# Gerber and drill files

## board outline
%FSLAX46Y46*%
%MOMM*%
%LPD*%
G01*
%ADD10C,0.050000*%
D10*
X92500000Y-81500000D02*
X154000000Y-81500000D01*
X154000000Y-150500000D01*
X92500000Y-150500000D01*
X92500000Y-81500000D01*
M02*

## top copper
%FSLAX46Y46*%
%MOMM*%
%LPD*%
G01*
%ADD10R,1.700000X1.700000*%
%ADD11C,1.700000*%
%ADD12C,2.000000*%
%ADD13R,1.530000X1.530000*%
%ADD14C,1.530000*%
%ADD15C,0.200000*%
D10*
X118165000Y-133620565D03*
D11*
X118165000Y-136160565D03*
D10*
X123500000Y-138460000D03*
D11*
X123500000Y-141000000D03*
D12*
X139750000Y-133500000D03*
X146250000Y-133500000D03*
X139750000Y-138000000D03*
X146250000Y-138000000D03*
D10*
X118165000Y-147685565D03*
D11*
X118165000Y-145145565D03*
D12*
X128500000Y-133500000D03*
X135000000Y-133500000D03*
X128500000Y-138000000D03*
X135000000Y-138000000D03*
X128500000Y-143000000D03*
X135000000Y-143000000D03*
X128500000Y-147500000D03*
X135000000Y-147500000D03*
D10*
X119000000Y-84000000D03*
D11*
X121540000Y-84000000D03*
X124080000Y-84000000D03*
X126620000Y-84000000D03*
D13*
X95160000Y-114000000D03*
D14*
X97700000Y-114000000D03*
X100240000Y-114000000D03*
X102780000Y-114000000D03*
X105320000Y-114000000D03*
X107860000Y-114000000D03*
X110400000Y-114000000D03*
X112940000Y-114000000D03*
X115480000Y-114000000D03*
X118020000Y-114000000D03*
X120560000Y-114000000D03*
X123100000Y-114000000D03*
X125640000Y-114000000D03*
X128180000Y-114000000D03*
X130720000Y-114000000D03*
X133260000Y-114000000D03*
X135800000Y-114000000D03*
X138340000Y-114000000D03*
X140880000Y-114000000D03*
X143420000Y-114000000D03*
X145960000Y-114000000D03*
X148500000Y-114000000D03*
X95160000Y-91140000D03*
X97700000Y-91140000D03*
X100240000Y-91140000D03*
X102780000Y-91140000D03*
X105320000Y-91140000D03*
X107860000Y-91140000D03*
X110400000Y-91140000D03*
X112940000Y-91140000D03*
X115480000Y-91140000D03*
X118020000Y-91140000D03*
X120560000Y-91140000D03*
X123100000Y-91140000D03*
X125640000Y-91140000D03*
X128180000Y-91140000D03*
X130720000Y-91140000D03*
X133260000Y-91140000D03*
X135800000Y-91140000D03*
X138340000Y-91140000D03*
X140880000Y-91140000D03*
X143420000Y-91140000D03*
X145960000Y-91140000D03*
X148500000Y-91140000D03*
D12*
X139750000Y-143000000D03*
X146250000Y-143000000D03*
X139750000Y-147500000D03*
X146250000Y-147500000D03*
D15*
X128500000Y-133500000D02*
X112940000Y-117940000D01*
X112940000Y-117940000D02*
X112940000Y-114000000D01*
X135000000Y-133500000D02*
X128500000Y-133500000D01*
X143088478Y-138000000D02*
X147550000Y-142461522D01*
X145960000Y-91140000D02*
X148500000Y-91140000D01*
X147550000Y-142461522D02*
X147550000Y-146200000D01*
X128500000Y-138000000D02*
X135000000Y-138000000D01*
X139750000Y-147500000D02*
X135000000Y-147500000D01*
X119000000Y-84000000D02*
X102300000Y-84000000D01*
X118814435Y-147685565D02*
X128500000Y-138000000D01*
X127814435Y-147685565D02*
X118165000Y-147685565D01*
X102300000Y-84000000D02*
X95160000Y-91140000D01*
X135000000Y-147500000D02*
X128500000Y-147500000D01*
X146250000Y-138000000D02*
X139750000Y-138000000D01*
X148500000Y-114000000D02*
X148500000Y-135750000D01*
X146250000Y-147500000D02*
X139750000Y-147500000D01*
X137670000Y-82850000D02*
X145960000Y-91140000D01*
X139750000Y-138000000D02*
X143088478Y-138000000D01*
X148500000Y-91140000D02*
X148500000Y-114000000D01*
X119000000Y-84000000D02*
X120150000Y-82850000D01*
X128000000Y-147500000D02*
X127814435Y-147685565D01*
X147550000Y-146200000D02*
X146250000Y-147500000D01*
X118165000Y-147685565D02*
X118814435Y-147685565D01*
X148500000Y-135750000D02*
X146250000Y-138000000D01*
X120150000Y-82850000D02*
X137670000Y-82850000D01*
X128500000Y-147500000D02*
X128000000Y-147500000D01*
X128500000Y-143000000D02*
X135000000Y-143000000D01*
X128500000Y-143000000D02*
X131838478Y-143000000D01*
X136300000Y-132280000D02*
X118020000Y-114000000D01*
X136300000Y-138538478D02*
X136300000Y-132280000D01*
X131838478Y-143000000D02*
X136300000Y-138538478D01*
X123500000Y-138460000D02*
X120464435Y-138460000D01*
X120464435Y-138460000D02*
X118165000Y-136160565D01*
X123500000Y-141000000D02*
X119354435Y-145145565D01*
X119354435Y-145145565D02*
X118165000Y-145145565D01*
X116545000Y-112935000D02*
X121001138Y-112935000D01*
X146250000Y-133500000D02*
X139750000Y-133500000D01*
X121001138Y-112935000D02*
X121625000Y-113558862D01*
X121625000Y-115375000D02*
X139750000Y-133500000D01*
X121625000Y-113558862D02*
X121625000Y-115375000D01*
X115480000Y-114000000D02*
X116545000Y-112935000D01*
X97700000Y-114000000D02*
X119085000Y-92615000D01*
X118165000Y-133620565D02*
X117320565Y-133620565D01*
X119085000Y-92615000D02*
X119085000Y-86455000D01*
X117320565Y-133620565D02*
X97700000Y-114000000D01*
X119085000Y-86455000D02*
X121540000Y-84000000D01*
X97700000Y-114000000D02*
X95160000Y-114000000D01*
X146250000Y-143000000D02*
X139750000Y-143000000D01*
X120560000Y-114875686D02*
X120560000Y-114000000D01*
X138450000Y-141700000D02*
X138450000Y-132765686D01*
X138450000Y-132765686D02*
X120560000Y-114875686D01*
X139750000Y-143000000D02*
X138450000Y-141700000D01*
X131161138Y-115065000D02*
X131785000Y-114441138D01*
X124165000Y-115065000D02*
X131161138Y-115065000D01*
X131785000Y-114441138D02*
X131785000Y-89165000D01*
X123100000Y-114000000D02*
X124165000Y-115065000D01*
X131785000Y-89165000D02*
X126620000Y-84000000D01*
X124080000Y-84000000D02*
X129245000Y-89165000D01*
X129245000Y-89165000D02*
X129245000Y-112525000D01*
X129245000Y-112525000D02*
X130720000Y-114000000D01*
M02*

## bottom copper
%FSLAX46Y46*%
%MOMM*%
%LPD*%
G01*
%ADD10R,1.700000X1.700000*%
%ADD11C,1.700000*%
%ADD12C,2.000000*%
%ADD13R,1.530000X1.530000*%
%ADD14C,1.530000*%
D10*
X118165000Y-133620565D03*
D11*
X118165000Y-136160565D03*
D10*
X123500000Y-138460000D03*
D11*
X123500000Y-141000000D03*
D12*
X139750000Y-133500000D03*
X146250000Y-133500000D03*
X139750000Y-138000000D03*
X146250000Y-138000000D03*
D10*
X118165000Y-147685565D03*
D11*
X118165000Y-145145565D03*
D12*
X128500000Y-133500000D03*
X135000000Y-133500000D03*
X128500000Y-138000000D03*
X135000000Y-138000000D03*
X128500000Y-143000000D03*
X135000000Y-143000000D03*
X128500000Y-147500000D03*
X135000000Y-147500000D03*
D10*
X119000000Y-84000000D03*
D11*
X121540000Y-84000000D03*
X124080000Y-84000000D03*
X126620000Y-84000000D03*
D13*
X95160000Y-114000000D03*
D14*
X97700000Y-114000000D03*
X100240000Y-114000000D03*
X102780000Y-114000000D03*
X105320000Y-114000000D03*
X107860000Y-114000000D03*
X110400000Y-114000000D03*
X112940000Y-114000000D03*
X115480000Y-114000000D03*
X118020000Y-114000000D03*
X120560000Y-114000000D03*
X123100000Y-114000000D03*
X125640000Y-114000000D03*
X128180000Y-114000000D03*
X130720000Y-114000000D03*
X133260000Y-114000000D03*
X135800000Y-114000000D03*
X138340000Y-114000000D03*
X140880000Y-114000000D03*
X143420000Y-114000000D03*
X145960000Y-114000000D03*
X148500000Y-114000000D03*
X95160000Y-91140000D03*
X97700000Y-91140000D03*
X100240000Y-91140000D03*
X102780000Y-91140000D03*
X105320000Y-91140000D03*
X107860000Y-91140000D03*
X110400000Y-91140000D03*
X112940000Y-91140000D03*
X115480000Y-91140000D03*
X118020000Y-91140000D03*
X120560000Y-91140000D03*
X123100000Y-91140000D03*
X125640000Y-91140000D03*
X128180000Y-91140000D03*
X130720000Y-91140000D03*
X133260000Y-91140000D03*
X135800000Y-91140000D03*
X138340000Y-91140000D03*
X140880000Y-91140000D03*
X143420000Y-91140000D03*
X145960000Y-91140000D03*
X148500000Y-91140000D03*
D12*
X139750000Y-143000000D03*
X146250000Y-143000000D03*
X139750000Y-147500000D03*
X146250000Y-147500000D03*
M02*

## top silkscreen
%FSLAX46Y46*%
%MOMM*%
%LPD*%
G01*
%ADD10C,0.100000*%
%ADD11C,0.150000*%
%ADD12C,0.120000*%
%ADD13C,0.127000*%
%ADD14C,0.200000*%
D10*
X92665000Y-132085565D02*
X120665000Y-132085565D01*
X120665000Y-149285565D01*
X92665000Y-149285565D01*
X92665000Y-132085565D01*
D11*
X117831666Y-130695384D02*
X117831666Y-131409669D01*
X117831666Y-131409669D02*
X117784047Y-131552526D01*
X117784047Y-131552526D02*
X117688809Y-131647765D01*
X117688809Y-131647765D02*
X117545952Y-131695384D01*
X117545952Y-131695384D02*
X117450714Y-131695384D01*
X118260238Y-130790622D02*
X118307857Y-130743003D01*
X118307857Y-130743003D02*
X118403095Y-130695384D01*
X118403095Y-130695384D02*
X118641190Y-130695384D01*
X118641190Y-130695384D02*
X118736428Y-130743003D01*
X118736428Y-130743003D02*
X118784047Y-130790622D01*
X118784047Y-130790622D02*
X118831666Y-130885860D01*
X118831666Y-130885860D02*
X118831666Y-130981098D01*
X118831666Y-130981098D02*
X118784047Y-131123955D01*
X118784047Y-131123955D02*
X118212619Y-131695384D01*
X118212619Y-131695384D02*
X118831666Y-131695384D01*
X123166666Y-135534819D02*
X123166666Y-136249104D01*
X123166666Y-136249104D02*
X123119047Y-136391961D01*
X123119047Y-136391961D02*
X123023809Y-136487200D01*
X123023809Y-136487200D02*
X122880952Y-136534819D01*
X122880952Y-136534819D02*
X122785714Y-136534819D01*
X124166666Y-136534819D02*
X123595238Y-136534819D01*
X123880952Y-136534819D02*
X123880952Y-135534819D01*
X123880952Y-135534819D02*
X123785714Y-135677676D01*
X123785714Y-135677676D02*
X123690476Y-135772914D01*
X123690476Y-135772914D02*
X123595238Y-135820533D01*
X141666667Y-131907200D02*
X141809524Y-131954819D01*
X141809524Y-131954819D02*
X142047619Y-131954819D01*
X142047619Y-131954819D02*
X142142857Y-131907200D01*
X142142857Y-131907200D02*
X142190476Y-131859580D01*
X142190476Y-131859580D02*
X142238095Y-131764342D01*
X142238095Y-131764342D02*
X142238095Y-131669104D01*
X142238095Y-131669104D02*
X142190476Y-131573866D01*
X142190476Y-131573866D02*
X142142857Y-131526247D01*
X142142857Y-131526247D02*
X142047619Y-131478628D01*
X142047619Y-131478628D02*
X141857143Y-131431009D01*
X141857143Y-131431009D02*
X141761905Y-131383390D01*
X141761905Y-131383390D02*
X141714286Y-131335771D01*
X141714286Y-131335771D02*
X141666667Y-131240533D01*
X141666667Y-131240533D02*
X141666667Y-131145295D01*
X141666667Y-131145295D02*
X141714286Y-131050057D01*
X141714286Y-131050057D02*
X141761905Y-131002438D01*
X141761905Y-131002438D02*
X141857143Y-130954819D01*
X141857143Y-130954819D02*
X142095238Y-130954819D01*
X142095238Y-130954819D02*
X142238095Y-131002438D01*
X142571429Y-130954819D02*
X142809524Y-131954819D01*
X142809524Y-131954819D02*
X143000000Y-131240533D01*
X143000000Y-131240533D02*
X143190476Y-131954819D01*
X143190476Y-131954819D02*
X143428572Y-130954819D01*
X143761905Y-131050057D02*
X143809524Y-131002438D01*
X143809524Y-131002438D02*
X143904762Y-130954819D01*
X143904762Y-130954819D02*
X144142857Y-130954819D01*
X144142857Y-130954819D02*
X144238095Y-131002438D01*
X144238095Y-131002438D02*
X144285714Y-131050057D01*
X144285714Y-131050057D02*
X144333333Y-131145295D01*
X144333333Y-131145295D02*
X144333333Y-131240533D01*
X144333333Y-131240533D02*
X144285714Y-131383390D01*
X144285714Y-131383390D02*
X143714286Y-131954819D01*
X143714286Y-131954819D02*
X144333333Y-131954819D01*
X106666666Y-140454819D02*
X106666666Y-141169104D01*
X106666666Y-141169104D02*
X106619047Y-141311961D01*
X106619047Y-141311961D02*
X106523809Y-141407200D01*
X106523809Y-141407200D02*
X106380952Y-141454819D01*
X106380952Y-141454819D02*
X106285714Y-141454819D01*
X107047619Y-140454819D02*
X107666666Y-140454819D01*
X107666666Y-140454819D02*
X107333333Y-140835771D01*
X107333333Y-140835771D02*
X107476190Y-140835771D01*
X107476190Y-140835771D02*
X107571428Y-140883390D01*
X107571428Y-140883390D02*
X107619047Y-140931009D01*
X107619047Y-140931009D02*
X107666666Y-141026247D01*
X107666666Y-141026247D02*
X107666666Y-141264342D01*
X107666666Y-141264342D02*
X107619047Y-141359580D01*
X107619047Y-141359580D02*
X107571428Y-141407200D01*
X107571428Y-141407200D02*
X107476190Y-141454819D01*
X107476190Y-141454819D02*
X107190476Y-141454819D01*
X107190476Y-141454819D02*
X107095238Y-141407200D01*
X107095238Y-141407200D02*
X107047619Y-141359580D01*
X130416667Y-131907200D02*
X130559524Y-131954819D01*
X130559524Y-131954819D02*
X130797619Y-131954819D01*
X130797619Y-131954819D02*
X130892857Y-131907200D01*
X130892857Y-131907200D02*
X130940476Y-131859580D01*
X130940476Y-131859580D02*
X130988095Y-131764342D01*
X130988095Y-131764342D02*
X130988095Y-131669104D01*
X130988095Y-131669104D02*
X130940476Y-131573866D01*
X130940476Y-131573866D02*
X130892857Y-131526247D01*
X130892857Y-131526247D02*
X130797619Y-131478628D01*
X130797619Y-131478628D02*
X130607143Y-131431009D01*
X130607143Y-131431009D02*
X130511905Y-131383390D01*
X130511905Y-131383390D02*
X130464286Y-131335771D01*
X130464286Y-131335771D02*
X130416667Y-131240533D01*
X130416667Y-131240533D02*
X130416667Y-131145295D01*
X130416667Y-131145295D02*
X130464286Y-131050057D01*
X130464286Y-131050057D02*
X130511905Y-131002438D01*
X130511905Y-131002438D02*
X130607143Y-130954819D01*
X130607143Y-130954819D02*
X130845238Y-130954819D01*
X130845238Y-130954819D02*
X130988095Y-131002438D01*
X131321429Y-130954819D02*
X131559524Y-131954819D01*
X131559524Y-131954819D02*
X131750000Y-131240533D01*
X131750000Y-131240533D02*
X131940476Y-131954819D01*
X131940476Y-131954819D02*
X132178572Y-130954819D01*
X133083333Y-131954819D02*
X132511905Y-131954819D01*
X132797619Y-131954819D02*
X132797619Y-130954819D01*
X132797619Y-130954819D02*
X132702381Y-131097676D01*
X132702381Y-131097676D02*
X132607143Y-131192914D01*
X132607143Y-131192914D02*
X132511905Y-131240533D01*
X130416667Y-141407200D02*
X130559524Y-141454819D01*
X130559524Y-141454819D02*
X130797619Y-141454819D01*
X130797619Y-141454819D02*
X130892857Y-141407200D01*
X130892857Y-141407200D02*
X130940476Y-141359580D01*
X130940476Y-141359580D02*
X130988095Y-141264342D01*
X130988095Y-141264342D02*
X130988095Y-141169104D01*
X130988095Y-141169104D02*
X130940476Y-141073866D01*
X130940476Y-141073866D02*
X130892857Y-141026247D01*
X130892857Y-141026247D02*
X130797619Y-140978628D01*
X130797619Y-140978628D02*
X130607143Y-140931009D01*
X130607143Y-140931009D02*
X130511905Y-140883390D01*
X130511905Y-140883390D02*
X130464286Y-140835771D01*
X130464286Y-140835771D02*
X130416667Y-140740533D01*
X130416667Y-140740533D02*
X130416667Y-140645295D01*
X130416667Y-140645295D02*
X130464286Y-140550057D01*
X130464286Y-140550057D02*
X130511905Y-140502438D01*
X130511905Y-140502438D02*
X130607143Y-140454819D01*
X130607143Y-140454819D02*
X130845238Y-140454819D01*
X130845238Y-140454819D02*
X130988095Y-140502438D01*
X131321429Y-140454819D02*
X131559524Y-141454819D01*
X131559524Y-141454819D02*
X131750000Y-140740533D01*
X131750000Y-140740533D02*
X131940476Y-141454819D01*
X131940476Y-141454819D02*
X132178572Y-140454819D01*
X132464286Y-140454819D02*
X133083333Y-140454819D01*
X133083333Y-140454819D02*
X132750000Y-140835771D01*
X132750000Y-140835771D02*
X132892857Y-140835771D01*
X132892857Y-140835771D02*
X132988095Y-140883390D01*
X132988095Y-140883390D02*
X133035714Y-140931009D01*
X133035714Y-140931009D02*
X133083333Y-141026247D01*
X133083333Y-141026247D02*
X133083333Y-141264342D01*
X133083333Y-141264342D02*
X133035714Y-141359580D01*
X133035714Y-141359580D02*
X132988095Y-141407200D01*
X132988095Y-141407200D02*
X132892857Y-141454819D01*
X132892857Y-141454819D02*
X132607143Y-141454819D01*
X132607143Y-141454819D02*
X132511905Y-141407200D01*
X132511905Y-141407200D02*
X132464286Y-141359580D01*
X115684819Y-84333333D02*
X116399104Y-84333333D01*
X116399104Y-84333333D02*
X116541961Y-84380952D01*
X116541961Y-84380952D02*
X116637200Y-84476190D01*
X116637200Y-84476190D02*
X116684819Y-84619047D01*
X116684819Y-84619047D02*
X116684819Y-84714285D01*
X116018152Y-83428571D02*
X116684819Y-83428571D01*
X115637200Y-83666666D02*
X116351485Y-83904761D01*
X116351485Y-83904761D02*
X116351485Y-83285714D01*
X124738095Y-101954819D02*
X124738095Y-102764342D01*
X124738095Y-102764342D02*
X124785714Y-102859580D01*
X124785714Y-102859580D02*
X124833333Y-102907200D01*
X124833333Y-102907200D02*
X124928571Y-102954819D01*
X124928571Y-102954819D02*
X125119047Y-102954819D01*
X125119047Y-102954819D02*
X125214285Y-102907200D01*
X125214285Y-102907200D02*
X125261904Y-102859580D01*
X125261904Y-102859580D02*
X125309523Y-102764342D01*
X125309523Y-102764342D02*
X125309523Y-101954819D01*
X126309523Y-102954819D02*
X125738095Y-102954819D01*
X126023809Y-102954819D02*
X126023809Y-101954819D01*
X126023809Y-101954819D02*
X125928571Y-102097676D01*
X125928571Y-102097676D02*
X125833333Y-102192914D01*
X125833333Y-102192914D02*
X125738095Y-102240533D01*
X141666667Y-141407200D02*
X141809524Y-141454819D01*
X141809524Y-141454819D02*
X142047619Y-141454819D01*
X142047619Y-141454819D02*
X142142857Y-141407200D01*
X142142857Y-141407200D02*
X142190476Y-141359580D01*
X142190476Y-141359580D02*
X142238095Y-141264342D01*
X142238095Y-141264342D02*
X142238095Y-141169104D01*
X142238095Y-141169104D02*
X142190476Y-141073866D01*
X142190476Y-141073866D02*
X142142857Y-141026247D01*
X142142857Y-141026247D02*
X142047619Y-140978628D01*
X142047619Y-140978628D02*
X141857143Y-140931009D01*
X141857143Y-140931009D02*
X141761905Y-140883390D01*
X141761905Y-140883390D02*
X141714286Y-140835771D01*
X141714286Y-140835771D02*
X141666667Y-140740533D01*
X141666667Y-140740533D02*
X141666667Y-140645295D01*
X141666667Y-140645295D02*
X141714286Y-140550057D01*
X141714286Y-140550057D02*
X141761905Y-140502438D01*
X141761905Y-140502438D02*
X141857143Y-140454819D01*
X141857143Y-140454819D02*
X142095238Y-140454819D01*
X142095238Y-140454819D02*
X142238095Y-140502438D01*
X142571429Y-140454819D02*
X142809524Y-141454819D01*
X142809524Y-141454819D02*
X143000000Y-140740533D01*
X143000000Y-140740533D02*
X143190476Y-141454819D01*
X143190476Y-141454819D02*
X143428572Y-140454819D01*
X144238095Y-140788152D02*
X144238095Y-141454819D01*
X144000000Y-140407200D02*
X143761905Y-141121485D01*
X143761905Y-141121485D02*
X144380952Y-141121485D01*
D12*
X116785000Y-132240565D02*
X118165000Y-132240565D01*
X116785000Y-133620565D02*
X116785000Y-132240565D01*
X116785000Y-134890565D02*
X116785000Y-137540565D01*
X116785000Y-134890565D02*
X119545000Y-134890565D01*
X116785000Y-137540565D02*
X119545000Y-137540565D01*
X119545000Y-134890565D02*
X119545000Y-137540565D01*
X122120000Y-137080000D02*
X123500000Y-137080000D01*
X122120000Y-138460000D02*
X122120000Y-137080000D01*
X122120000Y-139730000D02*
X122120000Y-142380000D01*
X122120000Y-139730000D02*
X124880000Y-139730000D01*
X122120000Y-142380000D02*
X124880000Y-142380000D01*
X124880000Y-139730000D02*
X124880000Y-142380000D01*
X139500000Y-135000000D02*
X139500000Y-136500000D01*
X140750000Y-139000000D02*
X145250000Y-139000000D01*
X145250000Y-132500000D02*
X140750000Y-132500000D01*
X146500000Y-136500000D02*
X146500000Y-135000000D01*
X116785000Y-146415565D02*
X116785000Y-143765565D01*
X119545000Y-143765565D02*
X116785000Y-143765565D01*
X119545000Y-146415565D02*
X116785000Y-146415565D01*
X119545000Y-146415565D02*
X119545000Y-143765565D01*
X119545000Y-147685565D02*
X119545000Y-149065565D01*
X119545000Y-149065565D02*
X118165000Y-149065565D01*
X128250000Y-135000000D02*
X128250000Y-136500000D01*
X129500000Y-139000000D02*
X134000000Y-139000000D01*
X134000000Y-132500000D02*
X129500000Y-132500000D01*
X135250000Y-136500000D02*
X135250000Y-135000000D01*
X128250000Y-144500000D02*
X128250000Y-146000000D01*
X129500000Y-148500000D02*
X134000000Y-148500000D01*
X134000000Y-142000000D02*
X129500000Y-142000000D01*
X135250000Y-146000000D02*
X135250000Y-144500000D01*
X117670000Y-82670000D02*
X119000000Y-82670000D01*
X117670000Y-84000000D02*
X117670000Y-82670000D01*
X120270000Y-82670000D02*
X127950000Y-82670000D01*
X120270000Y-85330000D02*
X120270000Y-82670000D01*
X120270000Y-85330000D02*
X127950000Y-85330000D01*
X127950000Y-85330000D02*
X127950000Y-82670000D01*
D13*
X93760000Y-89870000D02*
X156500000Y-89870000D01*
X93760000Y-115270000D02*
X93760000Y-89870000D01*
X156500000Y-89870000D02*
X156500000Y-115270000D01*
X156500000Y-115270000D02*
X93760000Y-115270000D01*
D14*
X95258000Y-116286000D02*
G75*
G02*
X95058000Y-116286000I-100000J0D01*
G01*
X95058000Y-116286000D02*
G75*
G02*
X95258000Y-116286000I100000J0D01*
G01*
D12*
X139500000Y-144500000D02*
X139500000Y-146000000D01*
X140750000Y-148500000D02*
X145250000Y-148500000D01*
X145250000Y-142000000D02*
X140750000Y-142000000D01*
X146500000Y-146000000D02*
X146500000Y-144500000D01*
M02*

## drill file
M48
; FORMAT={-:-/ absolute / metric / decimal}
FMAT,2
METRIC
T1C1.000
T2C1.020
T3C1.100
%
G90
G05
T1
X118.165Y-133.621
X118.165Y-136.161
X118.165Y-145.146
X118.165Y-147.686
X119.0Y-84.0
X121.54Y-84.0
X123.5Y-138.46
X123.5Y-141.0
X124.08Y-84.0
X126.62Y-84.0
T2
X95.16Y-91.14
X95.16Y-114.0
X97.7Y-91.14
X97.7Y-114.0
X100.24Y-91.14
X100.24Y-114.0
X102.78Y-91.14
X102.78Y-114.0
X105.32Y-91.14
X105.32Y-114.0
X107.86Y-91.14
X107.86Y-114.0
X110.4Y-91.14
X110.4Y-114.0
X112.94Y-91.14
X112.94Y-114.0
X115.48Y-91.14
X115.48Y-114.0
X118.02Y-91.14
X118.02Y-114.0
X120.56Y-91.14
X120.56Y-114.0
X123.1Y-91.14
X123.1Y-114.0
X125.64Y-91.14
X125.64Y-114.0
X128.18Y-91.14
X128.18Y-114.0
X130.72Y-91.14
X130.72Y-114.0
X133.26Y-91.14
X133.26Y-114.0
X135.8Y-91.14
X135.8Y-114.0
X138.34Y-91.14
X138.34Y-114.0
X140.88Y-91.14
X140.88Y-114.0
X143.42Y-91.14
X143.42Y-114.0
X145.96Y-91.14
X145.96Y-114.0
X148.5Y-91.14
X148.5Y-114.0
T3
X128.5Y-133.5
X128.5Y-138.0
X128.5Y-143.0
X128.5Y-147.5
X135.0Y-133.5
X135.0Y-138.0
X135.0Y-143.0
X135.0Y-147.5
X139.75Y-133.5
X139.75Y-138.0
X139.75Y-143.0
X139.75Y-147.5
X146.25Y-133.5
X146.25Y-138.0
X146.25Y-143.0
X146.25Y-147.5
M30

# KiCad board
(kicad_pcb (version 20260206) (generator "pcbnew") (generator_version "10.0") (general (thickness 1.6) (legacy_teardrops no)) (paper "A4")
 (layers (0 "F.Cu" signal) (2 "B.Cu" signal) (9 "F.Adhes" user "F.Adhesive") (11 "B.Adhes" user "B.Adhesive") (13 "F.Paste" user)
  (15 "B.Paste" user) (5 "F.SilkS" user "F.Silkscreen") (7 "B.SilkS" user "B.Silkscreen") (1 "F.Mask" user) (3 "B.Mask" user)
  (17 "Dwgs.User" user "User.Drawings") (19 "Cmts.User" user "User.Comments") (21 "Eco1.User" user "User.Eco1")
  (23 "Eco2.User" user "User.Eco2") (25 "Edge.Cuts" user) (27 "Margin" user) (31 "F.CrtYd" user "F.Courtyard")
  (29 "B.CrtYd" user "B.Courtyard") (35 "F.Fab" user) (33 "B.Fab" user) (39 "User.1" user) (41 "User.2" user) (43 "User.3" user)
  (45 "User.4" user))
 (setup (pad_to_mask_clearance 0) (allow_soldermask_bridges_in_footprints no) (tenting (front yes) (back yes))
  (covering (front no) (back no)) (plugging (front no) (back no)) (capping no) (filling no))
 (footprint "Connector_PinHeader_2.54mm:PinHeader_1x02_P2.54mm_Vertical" (layer "F.Cu") (at 118.165 133.620565)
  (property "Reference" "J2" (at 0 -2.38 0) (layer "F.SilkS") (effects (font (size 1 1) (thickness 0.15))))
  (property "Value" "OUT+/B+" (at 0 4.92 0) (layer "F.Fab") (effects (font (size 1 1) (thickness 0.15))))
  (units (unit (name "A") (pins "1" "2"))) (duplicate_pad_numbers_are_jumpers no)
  (fp_line (start -1.38 -1.38) (end 0 -1.38) (stroke (width 0.12) (type solid)) (layer "F.SilkS"))
  (fp_line (start -1.38 0) (end -1.38 -1.38) (stroke (width 0.12) (type solid)) (layer "F.SilkS"))
  (fp_line (start -1.38 1.27) (end -1.38 3.92) (stroke (width 0.12) (type solid)) (layer "F.SilkS"))
  (fp_line (start -1.38 1.27) (end 1.38 1.27) (stroke (width 0.12) (type solid)) (layer "F.SilkS"))
  (fp_line (start -1.38 3.92) (end 1.38 3.92) (stroke (width 0.12) (type solid)) (layer "F.SilkS"))
  (fp_line (start 1.38 1.27) (end 1.38 3.92) (stroke (width 0.12) (type solid)) (layer "F.SilkS"))
  (pad "1" thru_hole rect (at 0 0) (size 1.7 1.7) (drill 1) (layers "*.Cu" "*.Mask") (remove_unused_layers no) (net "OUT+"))
  (pad "2" thru_hole circle (at 0 2.54) (size 1.7 1.7) (drill 1) (layers "*.Cu" "*.Mask") (remove_unused_layers no) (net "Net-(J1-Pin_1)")))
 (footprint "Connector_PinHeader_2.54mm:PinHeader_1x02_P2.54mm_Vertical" (layer "F.Cu") (at 123.5 138.46)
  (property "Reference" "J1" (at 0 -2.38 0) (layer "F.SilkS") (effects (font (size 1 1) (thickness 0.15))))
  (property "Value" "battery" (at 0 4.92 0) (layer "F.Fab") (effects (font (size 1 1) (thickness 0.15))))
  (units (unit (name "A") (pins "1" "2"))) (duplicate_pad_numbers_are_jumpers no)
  (fp_line (start -1.38 -1.38) (end 0 -1.38) (stroke (width 0.12) (type solid)) (layer "F.SilkS"))
  (fp_line (start -1.38 0) (end -1.38 -1.38) (stroke (width 0.12) (type solid)) (layer "F.SilkS"))
  (fp_line (start -1.38 1.27) (end -1.38 3.92) (stroke (width 0.12) (type solid)) (layer "F.SilkS"))
  (fp_line (start -1.38 1.27) (end 1.38 1.27) (stroke (width 0.12) (type solid)) (layer "F.SilkS"))
  (fp_line (start -1.38 3.92) (end 1.38 3.92) (stroke (width 0.12) (type solid)) (layer "F.SilkS"))
  (fp_line (start 1.38 1.27) (end 1.38 3.92) (stroke (width 0.12) (type solid)) (layer "F.SilkS"))
  (pad "1" thru_hole rect (at 0 0) (size 1.7 1.7) (drill 1) (layers "*.Cu" "*.Mask") (remove_unused_layers no) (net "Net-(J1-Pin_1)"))
  (pad "2" thru_hole circle (at 0 2.54) (size 1.7 1.7) (drill 1) (layers "*.Cu" "*.Mask") (remove_unused_layers no) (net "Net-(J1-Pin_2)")))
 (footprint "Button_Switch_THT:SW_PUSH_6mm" (layer "F.Cu") (at 139.75 133.5)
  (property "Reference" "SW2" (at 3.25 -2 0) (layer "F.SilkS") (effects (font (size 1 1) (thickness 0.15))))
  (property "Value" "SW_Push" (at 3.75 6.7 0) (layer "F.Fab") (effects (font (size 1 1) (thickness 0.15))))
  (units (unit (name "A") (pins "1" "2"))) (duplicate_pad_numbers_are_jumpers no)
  (fp_line (start -0.25 1.5) (end -0.25 3) (stroke (width 0.12) (type solid)) (layer "F.SilkS"))
  (fp_line (start 1 5.5) (end 5.5 5.5) (stroke (width 0.12) (type solid)) (layer "F.SilkS"))
  (fp_line (start 5.5 -1) (end 1 -1) (stroke (width 0.12) (type solid)) (layer "F.SilkS"))
  (fp_line (start 6.75 3) (end 6.75 1.5) (stroke (width 0.12) (type solid)) (layer "F.SilkS"))
  (pad "1" thru_hole circle (at 0 0 90) (size 2 2) (drill 1.1) (layers "*.Cu" "*.Mask") (remove_unused_layers no) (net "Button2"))
  (pad "1" thru_hole circle (at 6.5 0 90) (size 2 2) (drill 1.1) (layers "*.Cu" "*.Mask") (remove_unused_layers no) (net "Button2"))
  (pad "2" thru_hole circle (at 0 4.5 90) (size 2 2) (drill 1.1) (layers "*.Cu" "*.Mask") (remove_unused_layers no) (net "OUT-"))
  (pad "2" thru_hole circle (at 6.5 4.5 90) (size 2 2) (drill 1.1) (layers "*.Cu" "*.Mask") (remove_unused_layers no) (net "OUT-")))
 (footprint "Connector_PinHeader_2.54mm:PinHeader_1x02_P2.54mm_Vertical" (layer "F.Cu") (at 118.165 147.685565 180)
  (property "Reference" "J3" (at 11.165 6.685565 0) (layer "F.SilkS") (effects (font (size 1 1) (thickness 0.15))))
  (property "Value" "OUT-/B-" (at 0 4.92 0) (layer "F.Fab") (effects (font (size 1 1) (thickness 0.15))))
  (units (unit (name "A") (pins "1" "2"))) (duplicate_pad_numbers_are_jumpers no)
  (fp_line (start 1.38 1.27) (end 1.38 3.92) (stroke (width 0.12) (type solid)) (layer "F.SilkS"))
  (fp_line (start -1.38 3.92) (end 1.38 3.92) (stroke (width 0.12) (type solid)) (layer "F.SilkS"))
  (fp_line (start -1.38 1.27) (end 1.38 1.27) (stroke (width 0.12) (type solid)) (layer "F.SilkS"))
  (fp_line (start -1.38 1.27) (end -1.38 3.92) (stroke (width 0.12) (type solid)) (layer "F.SilkS"))
  (fp_line (start -1.38 0) (end -1.38 -1.38) (stroke (width 0.12) (type solid)) (layer "F.SilkS"))
  (fp_line (start -1.38 -1.38) (end 0 -1.38) (stroke (width 0.12) (type solid)) (layer "F.SilkS"))
  (pad "1" thru_hole rect (at 0 0 180) (size 1.7 1.7) (drill 1) (layers "*.Cu" "*.Mask") (remove_unused_layers no) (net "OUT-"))
  (pad "2" thru_hole circle (at 0 2.54 180) (size 1.7 1.7) (drill 1) (layers "*.Cu" "*.Mask") (remove_unused_layers no)
   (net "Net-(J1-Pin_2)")))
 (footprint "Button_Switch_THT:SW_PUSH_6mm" (layer "F.Cu") (at 128.5 133.5)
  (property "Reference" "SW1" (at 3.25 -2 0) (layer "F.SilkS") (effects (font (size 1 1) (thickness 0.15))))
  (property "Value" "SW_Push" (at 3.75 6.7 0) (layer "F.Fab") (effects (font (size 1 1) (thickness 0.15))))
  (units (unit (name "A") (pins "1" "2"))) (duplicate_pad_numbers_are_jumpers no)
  (fp_line (start -0.25 1.5) (end -0.25 3) (stroke (width 0.12) (type solid)) (layer "F.SilkS"))
  (fp_line (start 1 5.5) (end 5.5 5.5) (stroke (width 0.12) (type solid)) (layer "F.SilkS"))
  (fp_line (start 5.5 -1) (end 1 -1) (stroke (width 0.12) (type solid)) (layer "F.SilkS"))
  (fp_line (start 6.75 3) (end 6.75 1.5) (stroke (width 0.12) (type solid)) (layer "F.SilkS"))
  (pad "1" thru_hole circle (at 0 0 90) (size 2 2) (drill 1.1) (layers "*.Cu" "*.Mask") (remove_unused_layers no) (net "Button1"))
  (pad "1" thru_hole circle (at 6.5 0 90) (size 2 2) (drill 1.1) (layers "*.Cu" "*.Mask") (remove_unused_layers no) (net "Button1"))
  (pad "2" thru_hole circle (at 0 4.5 90) (size 2 2) (drill 1.1) (layers "*.Cu" "*.Mask") (remove_unused_layers no) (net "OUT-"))
  (pad "2" thru_hole circle (at 6.5 4.5 90) (size 2 2) (drill 1.1) (layers "*.Cu" "*.Mask") (remove_unused_layers no) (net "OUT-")))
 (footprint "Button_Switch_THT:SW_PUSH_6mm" (layer "F.Cu") (at 128.5 143)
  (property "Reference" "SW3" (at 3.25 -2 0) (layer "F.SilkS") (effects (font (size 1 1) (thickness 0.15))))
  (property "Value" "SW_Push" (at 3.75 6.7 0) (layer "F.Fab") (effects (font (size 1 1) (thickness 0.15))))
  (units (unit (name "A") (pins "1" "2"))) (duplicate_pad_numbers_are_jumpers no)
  (fp_line (start -0.25 1.5) (end -0.25 3) (stroke (width 0.12) (type solid)) (layer "F.SilkS"))
  (fp_line (start 1 5.5) (end 5.5 5.5) (stroke (width 0.12) (type solid)) (layer "F.SilkS"))
  (fp_line (start 5.5 -1) (end 1 -1) (stroke (width 0.12) (type solid)) (layer "F.SilkS"))
  (fp_line (start 6.75 3) (end 6.75 1.5) (stroke (width 0.12) (type solid)) (layer "F.SilkS"))
  (pad "1" thru_hole circle (at 0 0 90) (size 2 2) (drill 1.1) (layers "*.Cu" "*.Mask") (remove_unused_layers no) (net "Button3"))
  (pad "1" thru_hole circle (at 6.5 0 90) (size 2 2) (drill 1.1) (layers "*.Cu" "*.Mask") (remove_unused_layers no) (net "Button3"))
  (pad "2" thru_hole circle (at 0 4.5 90) (size 2 2) (drill 1.1) (layers "*.Cu" "*.Mask") (remove_unused_layers no) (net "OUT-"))
  (pad "2" thru_hole circle (at 6.5 4.5 90) (size 2 2) (drill 1.1) (layers "*.Cu" "*.Mask") (remove_unused_layers no) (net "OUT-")))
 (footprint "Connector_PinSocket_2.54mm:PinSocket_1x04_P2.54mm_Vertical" (layer "F.Cu") (at 119 84 90)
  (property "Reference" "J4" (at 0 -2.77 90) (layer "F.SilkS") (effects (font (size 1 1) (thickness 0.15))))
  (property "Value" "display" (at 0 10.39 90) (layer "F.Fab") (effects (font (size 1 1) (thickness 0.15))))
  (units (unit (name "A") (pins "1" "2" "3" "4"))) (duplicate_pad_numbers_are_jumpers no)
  (fp_line (start 1.33 -1.33) (end 1.33 0) (stroke (width 0.12) (type solid)) (layer "F.SilkS"))
  (fp_line (start 0 -1.33) (end 1.33 -1.33) (stroke (width 0.12) (type solid)) (layer "F.SilkS"))
  (fp_line (start 1.33 1.27) (end 1.33 8.95) (stroke (width 0.12) (type solid)) (layer "F.SilkS"))
  (fp_line (start -1.33 1.27) (end 1.33 1.27) (stroke (width 0.12) (type solid)) (layer "F.SilkS"))
  (fp_line (start -1.33 1.27) (end -1.33 8.95) (stroke (width 0.12) (type solid)) (layer "F.SilkS"))
  (fp_line (start -1.33 8.95) (end 1.33 8.95) (stroke (width 0.12) (type solid)) (layer "F.SilkS"))
  (pad "1" thru_hole rect (at 0 0 90) (size 1.7 1.7) (drill 1) (layers "*.Cu" "*.Mask") (remove_unused_layers no) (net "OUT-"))
  (pad "2" thru_hole circle (at 0 2.54 90) (size 1.7 1.7) (drill 1) (layers "*.Cu" "*.Mask") (remove_unused_layers no) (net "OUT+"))
  (pad "3" thru_hole circle (at 0 5.08 90) (size 1.7 1.7) (drill 1) (layers "*.Cu" "*.Mask") (remove_unused_layers no) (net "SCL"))
  (pad "4" thru_hole circle (at 0 7.62 90) (size 1.7 1.7) (drill 1) (layers "*.Cu" "*.Mask") (remove_unused_layers no) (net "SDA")))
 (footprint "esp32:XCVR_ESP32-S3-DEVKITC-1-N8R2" (layer "F.Cu") (at 125.13 102.57 90)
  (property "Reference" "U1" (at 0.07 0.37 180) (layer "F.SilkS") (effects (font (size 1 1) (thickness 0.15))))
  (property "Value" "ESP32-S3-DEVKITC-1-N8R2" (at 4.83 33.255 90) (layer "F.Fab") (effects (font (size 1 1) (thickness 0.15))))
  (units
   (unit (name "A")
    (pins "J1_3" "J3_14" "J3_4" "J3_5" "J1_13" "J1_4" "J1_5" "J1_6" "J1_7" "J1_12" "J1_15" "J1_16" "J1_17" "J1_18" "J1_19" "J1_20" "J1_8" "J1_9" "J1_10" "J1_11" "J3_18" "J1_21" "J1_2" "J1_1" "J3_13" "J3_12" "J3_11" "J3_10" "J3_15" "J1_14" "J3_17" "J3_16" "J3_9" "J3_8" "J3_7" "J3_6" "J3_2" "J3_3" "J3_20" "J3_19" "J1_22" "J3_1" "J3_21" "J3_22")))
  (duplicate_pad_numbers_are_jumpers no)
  (fp_line (start 12.7 -31.37) (end 12.7 31.37) (stroke (width 0.127) (type solid)) (layer "F.SilkS"))
  (fp_line (start -12.7 -31.37) (end 12.7 -31.37) (stroke (width 0.127) (type solid)) (layer "F.SilkS"))
  (fp_line (start 12.7 31.37) (end -12.7 31.37) (stroke (width 0.127) (type solid)) (layer "F.SilkS"))
  (fp_line (start -12.7 31.37) (end -12.7 -31.37) (stroke (width 0.127) (type solid)) (layer "F.SilkS"))
  (fp_circle (center -13.716 -29.972) (end -13.616 -29.972) (stroke (width 0.2) (type solid)) (fill no) (layer "F.SilkS"))
  (pad "J1_1" thru_hole rect (at -11.43 -29.97 90) (size 1.53 1.53) (drill 1.02) (layers "*.Cu" "*.Mask") (remove_unused_layers no)
   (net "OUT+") (solder_mask_margin 0.102))
  (pad "J1_2" thru_hole circle (at -11.43 -27.43 90) (size 1.53 1.53) (drill 1.02) (layers "*.Cu" "*.Mask") (remove_unused_layers no)
   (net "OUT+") (solder_mask_margin 0.102))
  (pad "J1_3" thru_hole circle (at -11.43 -24.89 90) (size 1.53 1.53) (drill 1.02) (layers "*.Cu" "*.Mask") (remove_unused_layers no)
   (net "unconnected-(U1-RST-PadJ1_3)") (solder_mask_margin 0.102))
  (pad "J1_4" thru_hole circle (at -11.43 -22.35 90) (size 1.53 1.53) (drill 1.02) (layers "*.Cu" "*.Mask") (remove_unused_layers no)
   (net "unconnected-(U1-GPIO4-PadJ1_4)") (solder_mask_margin 0.102))
  (pad "J1_5" thru_hole circle (at -11.43 -19.81 90) (size 1.53 1.53) (drill 1.02) (layers "*.Cu" "*.Mask") (remove_unused_layers no)
   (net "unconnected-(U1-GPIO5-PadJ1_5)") (solder_mask_margin 0.102))
  (pad "J1_6" thru_hole circle (at -11.43 -17.27 90) (size 1.53 1.53) (drill 1.02) (layers "*.Cu" "*.Mask") (remove_unused_layers no)
   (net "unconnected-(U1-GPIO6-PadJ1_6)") (solder_mask_margin 0.102))
  (pad "J1_7" thru_hole circle (at -11.43 -14.73 90) (size 1.53 1.53) (drill 1.02) (layers "*.Cu" "*.Mask") (remove_unused_layers no)
   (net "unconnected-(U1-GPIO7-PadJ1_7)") (solder_mask_margin 0.102))
  (pad "J1_8" thru_hole circle (at -11.43 -12.19 90) (size 1.53 1.53) (drill 1.02) (layers "*.Cu" "*.Mask") (remove_unused_layers no)
   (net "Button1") (solder_mask_margin 0.102))
  (pad "J1_9" thru_hole circle (at -11.43 -9.65 90) (size 1.53 1.53) (drill 1.02) (layers "*.Cu" "*.Mask") (remove_unused_layers no)
   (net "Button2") (solder_mask_margin 0.102))
  (pad "J1_10" thru_hole circle (at -11.43 -7.11 90) (size 1.53 1.53) (drill 1.02) (layers "*.Cu" "*.Mask") (remove_unused_layers no)
   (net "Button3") (solder_mask_margin 0.102))
  (pad "J1_11" thru_hole circle (at -11.43 -4.57 90) (size 1.53 1.53) (drill 1.02) (layers "*.Cu" "*.Mask") (remove_unused_layers no)
   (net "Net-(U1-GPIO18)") (solder_mask_margin 0.102))
  (pad "J1_12" thru_hole circle (at -11.43 -2.03 90) (size 1.53 1.53) (drill 1.02) (layers "*.Cu" "*.Mask") (remove_unused_layers no)
   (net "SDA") (solder_mask_margin 0.102))
  (pad "J1_13" thru_hole circle (at -11.43 0.51 90) (size 1.53 1.53) (drill 1.02) (layers "*.Cu" "*.Mask") (remove_unused_layers no)
   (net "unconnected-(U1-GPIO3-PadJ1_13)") (solder_mask_margin 0.102))
  (pad "J1_14" thru_hole circle (at -11.43 3.05 90) (size 1.53 1.53) (drill 1.02) (layers "*.Cu" "*.Mask") (remove_unused_layers no)
   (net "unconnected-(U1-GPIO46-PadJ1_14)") (solder_mask_margin 0.102))
  (pad "J1_15" thru_hole circle (at -11.43 5.59 90) (size 1.53 1.53) (drill 1.02) (layers "*.Cu" "*.Mask") (remove_unused_layers no)
   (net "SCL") (solder_mask_margin 0.102))
  (pad "J1_16" thru_hole circle (at -11.43 8.13 90) (size 1.53 1.53) (drill 1.02) (layers "*.Cu" "*.Mask") (remove_unused_layers no)
   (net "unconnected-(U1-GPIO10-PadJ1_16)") (solder_mask_margin 0.102))
  (pad "J1_17" thru_hole circle (at -11.43 10.67 90) (size 1.53 1.53) (drill 1.02) (layers "*.Cu" "*.Mask") (remove_unused_layers no)
   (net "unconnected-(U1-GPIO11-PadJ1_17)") (solder_mask_margin 0.102))
  (pad "J1_18" thru_hole circle (at -11.43 13.21 90) (size 1.53 1.53) (drill 1.02) (layers "*.Cu" "*.Mask") (remove_unused_layers no)
   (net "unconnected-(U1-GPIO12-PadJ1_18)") (solder_mask_margin 0.102))
  (pad "J1_19" thru_hole circle (at -11.43 15.75 90) (size 1.53 1.53) (drill 1.02) (layers "*.Cu" "*.Mask") (remove_unused_layers no)
   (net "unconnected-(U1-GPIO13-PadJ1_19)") (solder_mask_margin 0.102))
  (pad "J1_20" thru_hole circle (at -11.43 18.29 90) (size 1.53 1.53) (drill 1.02) (layers "*.Cu" "*.Mask") (remove_unused_layers no)
   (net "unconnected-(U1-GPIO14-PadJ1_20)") (solder_mask_margin 0.102))
  (pad "J1_21" thru_hole circle (at -11.43 20.83 90) (size 1.53 1.53) (drill 1.02) (layers "*.Cu" "*.Mask") (remove_unused_layers no)
   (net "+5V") (solder_mask_margin 0.102))
  (pad "J1_22" thru_hole circle (at -11.43 23.37 90) (size 1.53 1.53) (drill 1.02) (layers "*.Cu" "*.Mask") (remove_unused_layers no)
   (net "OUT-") (solder_mask_margin 0.102))
  (pad "J3_1" thru_hole circle (at 11.43 -29.97 90) (size 1.53 1.53) (drill 1.02) (layers "*.Cu" "*.Mask") (remove_unused_layers no)
   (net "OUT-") (solder_mask_margin 0.102))
  (pad "J3_2" thru_hole circle (at 11.43 -27.43 90) (size 1.53 1.53) (drill 1.02) (layers "*.Cu" "*.Mask") (remove_unused_layers no)
   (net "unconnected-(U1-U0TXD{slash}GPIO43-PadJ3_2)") (solder_mask_margin 0.102))
  (pad "J3_3" thru_hole circle (at 11.43 -24.89 90) (size 1.53 1.53) (drill 1.02) (layers "*.Cu" "*.Mask") (remove_unused_layers no)
   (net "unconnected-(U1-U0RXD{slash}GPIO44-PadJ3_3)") (solder_mask_margin 0.102))
  (pad "J3_4" thru_hole circle (at 11.43 -22.35 90) (size 1.53 1.53) (drill 1.02) (layers "*.Cu" "*.Mask") (remove_unused_layers no)
   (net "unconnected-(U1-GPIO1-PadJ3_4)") (solder_mask_margin 0.102))
  (pad "J3_5" thru_hole circle (at 11.43 -19.81 90) (size 1.53 1.53) (drill 1.02) (layers "*.Cu" "*.Mask") (remove_unused_layers no)
   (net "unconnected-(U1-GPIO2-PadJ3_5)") (solder_mask_margin 0.102))
  (pad "J3_6" thru_hole circle (at 11.43 -17.27 90) (size 1.53 1.53) (drill 1.02) (layers "*.Cu" "*.Mask") (remove_unused_layers no)
   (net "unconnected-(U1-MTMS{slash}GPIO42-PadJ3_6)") (solder_mask_margin 0.102))
  (pad "J3_7" thru_hole circle (at 11.43 -14.73 90) (size 1.53 1.53) (drill 1.02) (layers "*.Cu" "*.Mask") (remove_unused_layers no)
   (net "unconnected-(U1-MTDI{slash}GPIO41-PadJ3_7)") (solder_mask_margin 0.102))
  (pad "J3_8" thru_hole circle (at 11.43 -12.19 90) (size 1.53 1.53) (drill 1.02) (layers "*.Cu" "*.Mask") (remove_unused_layers no)
   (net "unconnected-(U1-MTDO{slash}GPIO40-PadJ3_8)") (solder_mask_margin 0.102))
  (pad "J3_9" thru_hole circle (at 11.43 -9.65 90) (size 1.53 1.53) (drill 1.02) (layers "*.Cu" "*.Mask") (remove_unused_layers no)
   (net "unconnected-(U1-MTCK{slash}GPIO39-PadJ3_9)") (solder_mask_margin 0.102))
  (pad "J3_10" thru_hole circle (at 11.43 -7.11 90) (size 1.53 1.53) (drill 1.02) (layers "*.Cu" "*.Mask") (remove_unused_layers no)
   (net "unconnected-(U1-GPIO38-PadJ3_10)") (solder_mask_margin 0.102))
  (pad "J3_11" thru_hole circle (at 11.43 -4.57 90) (size 1.53 1.53) (drill 1.02) (layers "*.Cu" "*.Mask") (remove_unused_layers no)
   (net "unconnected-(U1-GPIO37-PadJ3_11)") (solder_mask_margin 0.102))
  (pad "J3_12" thru_hole circle (at 11.43 -2.03 90) (size 1.53 1.53) (drill 1.02) (layers "*.Cu" "*.Mask") (remove_unused_layers no)
   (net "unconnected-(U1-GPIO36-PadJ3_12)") (solder_mask_margin 0.102))
  (pad "J3_13" thru_hole circle (at 11.43 0.51 90) (size 1.53 1.53) (drill 1.02) (layers "*.Cu" "*.Mask") (remove_unused_layers no)
   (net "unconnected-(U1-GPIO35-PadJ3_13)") (solder_mask_margin 0.102))
  (pad "J3_14" thru_hole circle (at 11.43 3.05 90) (size 1.53 1.53) (drill 1.02) (layers "*.Cu" "*.Mask") (remove_unused_layers no)
   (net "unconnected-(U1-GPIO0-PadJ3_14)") (solder_mask_margin 0.102))
  (pad "J3_15" thru_hole circle (at 11.43 5.59 90) (size 1.53 1.53) (drill 1.02) (layers "*.Cu" "*.Mask") (remove_unused_layers no)
   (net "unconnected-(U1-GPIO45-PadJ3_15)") (solder_mask_margin 0.102))
  (pad "J3_16" thru_hole circle (at 11.43 8.13 90) (size 1.53 1.53) (drill 1.02) (layers "*.Cu" "*.Mask") (remove_unused_layers no)
   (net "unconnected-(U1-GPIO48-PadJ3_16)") (solder_mask_margin 0.102))
  (pad "J3_17" thru_hole circle (at 11.43 10.67 90) (size 1.53 1.53) (drill 1.02) (layers "*.Cu" "*.Mask") (remove_unused_layers no)
   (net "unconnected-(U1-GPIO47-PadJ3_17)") (solder_mask_margin 0.102))
  (pad "J3_18" thru_hole circle (at 11.43 13.21 90) (size 1.53 1.53) (drill 1.02) (layers "*.Cu" "*.Mask") (remove_unused_layers no)
   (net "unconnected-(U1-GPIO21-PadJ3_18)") (solder_mask_margin 0.102))
  (pad "J3_19" thru_hole circle (at 11.43 15.75 90) (size 1.53 1.53) (drill 1.02) (layers "*.Cu" "*.Mask") (remove_unused_layers no)
   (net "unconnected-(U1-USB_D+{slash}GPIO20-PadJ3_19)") (solder_mask_margin 0.102))
  (pad "J3_20" thru_hole circle (at 11.43 18.29 90) (size 1.53 1.53) (drill 1.02) (layers "*.Cu" "*.Mask") (remove_unused_layers no)
   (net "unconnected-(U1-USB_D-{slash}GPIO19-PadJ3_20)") (solder_mask_margin 0.102))
  (pad "J3_21" thru_hole circle (at 11.43 20.83 90) (size 1.53 1.53) (drill 1.02) (layers "*.Cu" "*.Mask") (remove_unused_layers no)
   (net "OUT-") (solder_mask_margin 0.102))
  (pad "J3_22" thru_hole circle (at 11.43 23.37 90) (size 1.53 1.53) (drill 1.02) (layers "*.Cu" "*.Mask") (remove_unused_layers no)
   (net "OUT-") (solder_mask_margin 0.102)))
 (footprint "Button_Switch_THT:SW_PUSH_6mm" (layer "F.Cu") (at 139.75 143)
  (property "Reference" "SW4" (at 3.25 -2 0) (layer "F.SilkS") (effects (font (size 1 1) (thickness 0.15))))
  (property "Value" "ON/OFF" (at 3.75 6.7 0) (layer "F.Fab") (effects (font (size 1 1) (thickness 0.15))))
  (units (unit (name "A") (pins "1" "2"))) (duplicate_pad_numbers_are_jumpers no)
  (fp_line (start -0.25 1.5) (end -0.25 3) (stroke (width 0.12) (type solid)) (layer "F.SilkS"))
  (fp_line (start 1 5.5) (end 5.5 5.5) (stroke (width 0.12) (type solid)) (layer "F.SilkS"))
  (fp_line (start 5.5 -1) (end 1 -1) (stroke (width 0.12) (type solid)) (layer "F.SilkS"))
  (fp_line (start 6.75 3) (end 6.75 1.5) (stroke (width 0.12) (type solid)) (layer "F.SilkS"))
  (pad "1" thru_hole circle (at 0 0 90) (size 2 2) (drill 1.1) (layers "*.Cu" "*.Mask") (remove_unused_layers no) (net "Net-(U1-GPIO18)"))
  (pad "1" thru_hole circle (at 6.5 0 90) (size 2 2) (drill 1.1) (layers "*.Cu" "*.Mask") (remove_unused_layers no) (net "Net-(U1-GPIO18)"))
  (pad "2" thru_hole circle (at 0 4.5 90) (size 2 2) (drill 1.1) (layers "*.Cu" "*.Mask") (remove_unused_layers no) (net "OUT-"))
  (pad "2" thru_hole circle (at 6.5 4.5 90) (size 2 2) (drill 1.1) (layers "*.Cu" "*.Mask") (remove_unused_layers no) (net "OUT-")))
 (gr_rect (start 92.665 132.085565) (end 120.665 149.285565) (stroke (width 0.1) (type solid)) (fill no) (layer "F.SilkS"))
 (gr_rect (start 92.5 81.5) (end 154 150.5) (stroke (width 0.05) (type default)) (fill no) (layer "Edge.Cuts"))
 (segment (start 128.5 133.5) (end 112.94 117.94) (width 0.2) (layer "F.Cu") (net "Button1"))
 (segment (start 112.94 117.94) (end 112.94 114) (width 0.2) (layer "F.Cu") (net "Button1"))
 (segment (start 135 133.5) (end 128.5 133.5) (width 0.2) (layer "F.Cu") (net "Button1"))
 (segment (start 143.088478 138) (end 147.55 142.461522) (width 0.2) (layer "F.Cu") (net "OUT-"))
 (segment (start 145.96 91.14) (end 148.5 91.14) (width 0.2) (layer "F.Cu") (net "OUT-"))
 (segment (start 147.55 142.461522) (end 147.55 146.2) (width 0.2) (layer "F.Cu") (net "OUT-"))
 (segment (start 128.5 138) (end 135 138) (width 0.2) (layer "F.Cu") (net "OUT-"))
 (segment (start 139.75 147.5) (end 135 147.5) (width 0.2) (layer "F.Cu") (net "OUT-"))
 (segment (start 119 84) (end 102.3 84) (width 0.2) (layer "F.Cu") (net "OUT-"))
 (segment (start 118.814435 147.685565) (end 128.5 138) (width 0.2) (layer "F.Cu") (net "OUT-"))
 (segment (start 127.814435 147.685565) (end 118.165 147.685565) (width 0.2) (layer "F.Cu") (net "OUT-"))
 (segment (start 102.3 84) (end 95.16 91.14) (width 0.2) (layer "F.Cu") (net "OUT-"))
 (segment (start 135 147.5) (end 128.5 147.5) (width 0.2) (layer "F.Cu") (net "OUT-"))
 (segment (start 146.25 138) (end 139.75 138) (width 0.2) (layer "F.Cu") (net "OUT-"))
 (segment (start 148.5 114) (end 148.5 135.75) (width 0.2) (layer "F.Cu") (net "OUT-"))
 (segment (start 146.25 147.5) (end 139.75 147.5) (width 0.2) (layer "F.Cu") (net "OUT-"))
 (segment (start 137.67 82.85) (end 145.96 91.14) (width 0.2) (layer "F.Cu") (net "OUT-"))
 (segment (start 139.75 138) (end 143.088478 138) (width 0.2) (layer "F.Cu") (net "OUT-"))
 (segment (start 148.5 91.14) (end 148.5 114) (width 0.2) (layer "F.Cu") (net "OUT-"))
 (segment (start 119 84) (end 120.15 82.85) (width 0.2) (layer "F.Cu") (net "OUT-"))
 (segment (start 128 147.5) (end 127.814435 147.685565) (width 0.2) (layer "F.Cu") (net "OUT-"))
 (segment (start 147.55 146.2) (end 146.25 147.5) (width 0.2) (layer "F.Cu") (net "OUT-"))
 (segment (start 118.165 147.685565) (end 118.814435 147.685565) (width 0.2) (layer "F.Cu") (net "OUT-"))
 (segment (start 148.5 135.75) (end 146.25 138) (width 0.2) (layer "F.Cu") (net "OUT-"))
 (segment (start 120.15 82.85) (end 137.67 82.85) (width 0.2) (layer "F.Cu") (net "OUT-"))
 (segment (start 128.5 147.5) (end 128 147.5) (width 0.2) (layer "F.Cu") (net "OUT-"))
 (segment (start 128.5 143) (end 135 143) (width 0.2) (layer "F.Cu") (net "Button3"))
 (segment (start 128.5 143) (end 131.838478 143) (width 0.2) (layer "F.Cu") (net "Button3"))
 (segment (start 136.3 132.28) (end 118.02 114) (width 0.2) (layer "F.Cu") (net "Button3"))
 (segment (start 136.3 138.538478) (end 136.3 132.28) (width 0.2) (layer "F.Cu") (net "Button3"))
 (segment (start 131.838478 143) (end 136.3 138.538478) (width 0.2) (layer "F.Cu") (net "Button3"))
 (segment (start 123.5 138.46) (end 120.464435 138.46) (width 0.2) (layer "F.Cu") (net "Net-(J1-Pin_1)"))
 (segment (start 120.464435 138.46) (end 118.165 136.160565) (width 0.2) (layer "F.Cu") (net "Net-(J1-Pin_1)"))
 (segment (start 123.5 141) (end 119.354435 145.145565) (width 0.2) (layer "F.Cu") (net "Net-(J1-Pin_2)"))
 (segment (start 119.354435 145.145565) (end 118.165 145.145565) (width 0.2) (layer "F.Cu") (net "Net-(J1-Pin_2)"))
 (segment (start 116.545 112.935) (end 121.001138 112.935) (width 0.2) (layer "F.Cu") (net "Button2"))
 (segment (start 146.25 133.5) (end 139.75 133.5) (width 0.2) (layer "F.Cu") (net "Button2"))
 (segment (start 121.001138 112.935) (end 121.625 113.558862) (width 0.2) (layer "F.Cu") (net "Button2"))
 (segment (start 121.625 115.375) (end 139.75 133.5) (width 0.2) (layer "F.Cu") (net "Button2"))
 (segment (start 121.625 113.558862) (end 121.625 115.375) (width 0.2) (layer "F.Cu") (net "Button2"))
 (segment (start 115.48 114) (end 116.545 112.935) (width 0.2) (layer "F.Cu") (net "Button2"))
 (segment (start 97.7 114) (end 119.085 92.615) (width 0.2) (layer "F.Cu") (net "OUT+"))
 (segment (start 118.165 133.620565) (end 117.320565 133.620565) (width 0.2) (layer "F.Cu") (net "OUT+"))
 (segment (start 119.085 92.615) (end 119.085 86.455) (width 0.2) (layer "F.Cu") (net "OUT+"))
 (segment (start 117.320565 133.620565) (end 97.7 114) (width 0.2) (layer "F.Cu") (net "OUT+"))
 (segment (start 119.085 86.455) (end 121.54 84) (width 0.2) (layer "F.Cu") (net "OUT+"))
 (segment (start 97.7 114) (end 95.16 114) (width 0.2) (layer "F.Cu") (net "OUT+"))
 (segment (start 146.25 143) (end 139.75 143) (width 0.2) (layer "F.Cu") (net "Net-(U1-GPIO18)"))
 (segment (start 120.56 114.875686) (end 120.56 114) (width 0.2) (layer "F.Cu") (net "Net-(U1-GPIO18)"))
 (segment (start 138.45 141.7) (end 138.45 132.765686) (width 0.2) (layer "F.Cu") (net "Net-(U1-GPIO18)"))
 (segment (start 138.45 132.765686) (end 120.56 114.875686) (width 0.2) (layer "F.Cu") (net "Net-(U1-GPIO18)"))
 (segment (start 139.75 143) (end 138.45 141.7) (width 0.2) (layer "F.Cu") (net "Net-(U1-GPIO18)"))
 (segment (start 131.161138 115.065) (end 131.785 114.441138) (width 0.2) (layer "F.Cu") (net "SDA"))
 (segment (start 124.165 115.065) (end 131.161138 115.065) (width 0.2) (layer "F.Cu") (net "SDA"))
 (segment (start 131.785 114.441138) (end 131.785 89.165) (width 0.2) (layer "F.Cu") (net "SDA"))
 (segment (start 123.1 114) (end 124.165 115.065) (width 0.2) (layer "F.Cu") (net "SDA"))
 (segment (start 131.785 89.165) (end 126.62 84) (width 0.2) (layer "F.Cu") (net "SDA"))
 (segment (start 124.08 84) (end 129.245 89.165) (width 0.2) (layer "F.Cu") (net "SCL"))
 (segment (start 129.245 89.165) (end 129.245 112.525) (width 0.2) (layer "F.Cu") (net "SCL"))
 (segment (start 129.245 112.525) (end 130.72 114) (width 0.2) (layer "F.Cu") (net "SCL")))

